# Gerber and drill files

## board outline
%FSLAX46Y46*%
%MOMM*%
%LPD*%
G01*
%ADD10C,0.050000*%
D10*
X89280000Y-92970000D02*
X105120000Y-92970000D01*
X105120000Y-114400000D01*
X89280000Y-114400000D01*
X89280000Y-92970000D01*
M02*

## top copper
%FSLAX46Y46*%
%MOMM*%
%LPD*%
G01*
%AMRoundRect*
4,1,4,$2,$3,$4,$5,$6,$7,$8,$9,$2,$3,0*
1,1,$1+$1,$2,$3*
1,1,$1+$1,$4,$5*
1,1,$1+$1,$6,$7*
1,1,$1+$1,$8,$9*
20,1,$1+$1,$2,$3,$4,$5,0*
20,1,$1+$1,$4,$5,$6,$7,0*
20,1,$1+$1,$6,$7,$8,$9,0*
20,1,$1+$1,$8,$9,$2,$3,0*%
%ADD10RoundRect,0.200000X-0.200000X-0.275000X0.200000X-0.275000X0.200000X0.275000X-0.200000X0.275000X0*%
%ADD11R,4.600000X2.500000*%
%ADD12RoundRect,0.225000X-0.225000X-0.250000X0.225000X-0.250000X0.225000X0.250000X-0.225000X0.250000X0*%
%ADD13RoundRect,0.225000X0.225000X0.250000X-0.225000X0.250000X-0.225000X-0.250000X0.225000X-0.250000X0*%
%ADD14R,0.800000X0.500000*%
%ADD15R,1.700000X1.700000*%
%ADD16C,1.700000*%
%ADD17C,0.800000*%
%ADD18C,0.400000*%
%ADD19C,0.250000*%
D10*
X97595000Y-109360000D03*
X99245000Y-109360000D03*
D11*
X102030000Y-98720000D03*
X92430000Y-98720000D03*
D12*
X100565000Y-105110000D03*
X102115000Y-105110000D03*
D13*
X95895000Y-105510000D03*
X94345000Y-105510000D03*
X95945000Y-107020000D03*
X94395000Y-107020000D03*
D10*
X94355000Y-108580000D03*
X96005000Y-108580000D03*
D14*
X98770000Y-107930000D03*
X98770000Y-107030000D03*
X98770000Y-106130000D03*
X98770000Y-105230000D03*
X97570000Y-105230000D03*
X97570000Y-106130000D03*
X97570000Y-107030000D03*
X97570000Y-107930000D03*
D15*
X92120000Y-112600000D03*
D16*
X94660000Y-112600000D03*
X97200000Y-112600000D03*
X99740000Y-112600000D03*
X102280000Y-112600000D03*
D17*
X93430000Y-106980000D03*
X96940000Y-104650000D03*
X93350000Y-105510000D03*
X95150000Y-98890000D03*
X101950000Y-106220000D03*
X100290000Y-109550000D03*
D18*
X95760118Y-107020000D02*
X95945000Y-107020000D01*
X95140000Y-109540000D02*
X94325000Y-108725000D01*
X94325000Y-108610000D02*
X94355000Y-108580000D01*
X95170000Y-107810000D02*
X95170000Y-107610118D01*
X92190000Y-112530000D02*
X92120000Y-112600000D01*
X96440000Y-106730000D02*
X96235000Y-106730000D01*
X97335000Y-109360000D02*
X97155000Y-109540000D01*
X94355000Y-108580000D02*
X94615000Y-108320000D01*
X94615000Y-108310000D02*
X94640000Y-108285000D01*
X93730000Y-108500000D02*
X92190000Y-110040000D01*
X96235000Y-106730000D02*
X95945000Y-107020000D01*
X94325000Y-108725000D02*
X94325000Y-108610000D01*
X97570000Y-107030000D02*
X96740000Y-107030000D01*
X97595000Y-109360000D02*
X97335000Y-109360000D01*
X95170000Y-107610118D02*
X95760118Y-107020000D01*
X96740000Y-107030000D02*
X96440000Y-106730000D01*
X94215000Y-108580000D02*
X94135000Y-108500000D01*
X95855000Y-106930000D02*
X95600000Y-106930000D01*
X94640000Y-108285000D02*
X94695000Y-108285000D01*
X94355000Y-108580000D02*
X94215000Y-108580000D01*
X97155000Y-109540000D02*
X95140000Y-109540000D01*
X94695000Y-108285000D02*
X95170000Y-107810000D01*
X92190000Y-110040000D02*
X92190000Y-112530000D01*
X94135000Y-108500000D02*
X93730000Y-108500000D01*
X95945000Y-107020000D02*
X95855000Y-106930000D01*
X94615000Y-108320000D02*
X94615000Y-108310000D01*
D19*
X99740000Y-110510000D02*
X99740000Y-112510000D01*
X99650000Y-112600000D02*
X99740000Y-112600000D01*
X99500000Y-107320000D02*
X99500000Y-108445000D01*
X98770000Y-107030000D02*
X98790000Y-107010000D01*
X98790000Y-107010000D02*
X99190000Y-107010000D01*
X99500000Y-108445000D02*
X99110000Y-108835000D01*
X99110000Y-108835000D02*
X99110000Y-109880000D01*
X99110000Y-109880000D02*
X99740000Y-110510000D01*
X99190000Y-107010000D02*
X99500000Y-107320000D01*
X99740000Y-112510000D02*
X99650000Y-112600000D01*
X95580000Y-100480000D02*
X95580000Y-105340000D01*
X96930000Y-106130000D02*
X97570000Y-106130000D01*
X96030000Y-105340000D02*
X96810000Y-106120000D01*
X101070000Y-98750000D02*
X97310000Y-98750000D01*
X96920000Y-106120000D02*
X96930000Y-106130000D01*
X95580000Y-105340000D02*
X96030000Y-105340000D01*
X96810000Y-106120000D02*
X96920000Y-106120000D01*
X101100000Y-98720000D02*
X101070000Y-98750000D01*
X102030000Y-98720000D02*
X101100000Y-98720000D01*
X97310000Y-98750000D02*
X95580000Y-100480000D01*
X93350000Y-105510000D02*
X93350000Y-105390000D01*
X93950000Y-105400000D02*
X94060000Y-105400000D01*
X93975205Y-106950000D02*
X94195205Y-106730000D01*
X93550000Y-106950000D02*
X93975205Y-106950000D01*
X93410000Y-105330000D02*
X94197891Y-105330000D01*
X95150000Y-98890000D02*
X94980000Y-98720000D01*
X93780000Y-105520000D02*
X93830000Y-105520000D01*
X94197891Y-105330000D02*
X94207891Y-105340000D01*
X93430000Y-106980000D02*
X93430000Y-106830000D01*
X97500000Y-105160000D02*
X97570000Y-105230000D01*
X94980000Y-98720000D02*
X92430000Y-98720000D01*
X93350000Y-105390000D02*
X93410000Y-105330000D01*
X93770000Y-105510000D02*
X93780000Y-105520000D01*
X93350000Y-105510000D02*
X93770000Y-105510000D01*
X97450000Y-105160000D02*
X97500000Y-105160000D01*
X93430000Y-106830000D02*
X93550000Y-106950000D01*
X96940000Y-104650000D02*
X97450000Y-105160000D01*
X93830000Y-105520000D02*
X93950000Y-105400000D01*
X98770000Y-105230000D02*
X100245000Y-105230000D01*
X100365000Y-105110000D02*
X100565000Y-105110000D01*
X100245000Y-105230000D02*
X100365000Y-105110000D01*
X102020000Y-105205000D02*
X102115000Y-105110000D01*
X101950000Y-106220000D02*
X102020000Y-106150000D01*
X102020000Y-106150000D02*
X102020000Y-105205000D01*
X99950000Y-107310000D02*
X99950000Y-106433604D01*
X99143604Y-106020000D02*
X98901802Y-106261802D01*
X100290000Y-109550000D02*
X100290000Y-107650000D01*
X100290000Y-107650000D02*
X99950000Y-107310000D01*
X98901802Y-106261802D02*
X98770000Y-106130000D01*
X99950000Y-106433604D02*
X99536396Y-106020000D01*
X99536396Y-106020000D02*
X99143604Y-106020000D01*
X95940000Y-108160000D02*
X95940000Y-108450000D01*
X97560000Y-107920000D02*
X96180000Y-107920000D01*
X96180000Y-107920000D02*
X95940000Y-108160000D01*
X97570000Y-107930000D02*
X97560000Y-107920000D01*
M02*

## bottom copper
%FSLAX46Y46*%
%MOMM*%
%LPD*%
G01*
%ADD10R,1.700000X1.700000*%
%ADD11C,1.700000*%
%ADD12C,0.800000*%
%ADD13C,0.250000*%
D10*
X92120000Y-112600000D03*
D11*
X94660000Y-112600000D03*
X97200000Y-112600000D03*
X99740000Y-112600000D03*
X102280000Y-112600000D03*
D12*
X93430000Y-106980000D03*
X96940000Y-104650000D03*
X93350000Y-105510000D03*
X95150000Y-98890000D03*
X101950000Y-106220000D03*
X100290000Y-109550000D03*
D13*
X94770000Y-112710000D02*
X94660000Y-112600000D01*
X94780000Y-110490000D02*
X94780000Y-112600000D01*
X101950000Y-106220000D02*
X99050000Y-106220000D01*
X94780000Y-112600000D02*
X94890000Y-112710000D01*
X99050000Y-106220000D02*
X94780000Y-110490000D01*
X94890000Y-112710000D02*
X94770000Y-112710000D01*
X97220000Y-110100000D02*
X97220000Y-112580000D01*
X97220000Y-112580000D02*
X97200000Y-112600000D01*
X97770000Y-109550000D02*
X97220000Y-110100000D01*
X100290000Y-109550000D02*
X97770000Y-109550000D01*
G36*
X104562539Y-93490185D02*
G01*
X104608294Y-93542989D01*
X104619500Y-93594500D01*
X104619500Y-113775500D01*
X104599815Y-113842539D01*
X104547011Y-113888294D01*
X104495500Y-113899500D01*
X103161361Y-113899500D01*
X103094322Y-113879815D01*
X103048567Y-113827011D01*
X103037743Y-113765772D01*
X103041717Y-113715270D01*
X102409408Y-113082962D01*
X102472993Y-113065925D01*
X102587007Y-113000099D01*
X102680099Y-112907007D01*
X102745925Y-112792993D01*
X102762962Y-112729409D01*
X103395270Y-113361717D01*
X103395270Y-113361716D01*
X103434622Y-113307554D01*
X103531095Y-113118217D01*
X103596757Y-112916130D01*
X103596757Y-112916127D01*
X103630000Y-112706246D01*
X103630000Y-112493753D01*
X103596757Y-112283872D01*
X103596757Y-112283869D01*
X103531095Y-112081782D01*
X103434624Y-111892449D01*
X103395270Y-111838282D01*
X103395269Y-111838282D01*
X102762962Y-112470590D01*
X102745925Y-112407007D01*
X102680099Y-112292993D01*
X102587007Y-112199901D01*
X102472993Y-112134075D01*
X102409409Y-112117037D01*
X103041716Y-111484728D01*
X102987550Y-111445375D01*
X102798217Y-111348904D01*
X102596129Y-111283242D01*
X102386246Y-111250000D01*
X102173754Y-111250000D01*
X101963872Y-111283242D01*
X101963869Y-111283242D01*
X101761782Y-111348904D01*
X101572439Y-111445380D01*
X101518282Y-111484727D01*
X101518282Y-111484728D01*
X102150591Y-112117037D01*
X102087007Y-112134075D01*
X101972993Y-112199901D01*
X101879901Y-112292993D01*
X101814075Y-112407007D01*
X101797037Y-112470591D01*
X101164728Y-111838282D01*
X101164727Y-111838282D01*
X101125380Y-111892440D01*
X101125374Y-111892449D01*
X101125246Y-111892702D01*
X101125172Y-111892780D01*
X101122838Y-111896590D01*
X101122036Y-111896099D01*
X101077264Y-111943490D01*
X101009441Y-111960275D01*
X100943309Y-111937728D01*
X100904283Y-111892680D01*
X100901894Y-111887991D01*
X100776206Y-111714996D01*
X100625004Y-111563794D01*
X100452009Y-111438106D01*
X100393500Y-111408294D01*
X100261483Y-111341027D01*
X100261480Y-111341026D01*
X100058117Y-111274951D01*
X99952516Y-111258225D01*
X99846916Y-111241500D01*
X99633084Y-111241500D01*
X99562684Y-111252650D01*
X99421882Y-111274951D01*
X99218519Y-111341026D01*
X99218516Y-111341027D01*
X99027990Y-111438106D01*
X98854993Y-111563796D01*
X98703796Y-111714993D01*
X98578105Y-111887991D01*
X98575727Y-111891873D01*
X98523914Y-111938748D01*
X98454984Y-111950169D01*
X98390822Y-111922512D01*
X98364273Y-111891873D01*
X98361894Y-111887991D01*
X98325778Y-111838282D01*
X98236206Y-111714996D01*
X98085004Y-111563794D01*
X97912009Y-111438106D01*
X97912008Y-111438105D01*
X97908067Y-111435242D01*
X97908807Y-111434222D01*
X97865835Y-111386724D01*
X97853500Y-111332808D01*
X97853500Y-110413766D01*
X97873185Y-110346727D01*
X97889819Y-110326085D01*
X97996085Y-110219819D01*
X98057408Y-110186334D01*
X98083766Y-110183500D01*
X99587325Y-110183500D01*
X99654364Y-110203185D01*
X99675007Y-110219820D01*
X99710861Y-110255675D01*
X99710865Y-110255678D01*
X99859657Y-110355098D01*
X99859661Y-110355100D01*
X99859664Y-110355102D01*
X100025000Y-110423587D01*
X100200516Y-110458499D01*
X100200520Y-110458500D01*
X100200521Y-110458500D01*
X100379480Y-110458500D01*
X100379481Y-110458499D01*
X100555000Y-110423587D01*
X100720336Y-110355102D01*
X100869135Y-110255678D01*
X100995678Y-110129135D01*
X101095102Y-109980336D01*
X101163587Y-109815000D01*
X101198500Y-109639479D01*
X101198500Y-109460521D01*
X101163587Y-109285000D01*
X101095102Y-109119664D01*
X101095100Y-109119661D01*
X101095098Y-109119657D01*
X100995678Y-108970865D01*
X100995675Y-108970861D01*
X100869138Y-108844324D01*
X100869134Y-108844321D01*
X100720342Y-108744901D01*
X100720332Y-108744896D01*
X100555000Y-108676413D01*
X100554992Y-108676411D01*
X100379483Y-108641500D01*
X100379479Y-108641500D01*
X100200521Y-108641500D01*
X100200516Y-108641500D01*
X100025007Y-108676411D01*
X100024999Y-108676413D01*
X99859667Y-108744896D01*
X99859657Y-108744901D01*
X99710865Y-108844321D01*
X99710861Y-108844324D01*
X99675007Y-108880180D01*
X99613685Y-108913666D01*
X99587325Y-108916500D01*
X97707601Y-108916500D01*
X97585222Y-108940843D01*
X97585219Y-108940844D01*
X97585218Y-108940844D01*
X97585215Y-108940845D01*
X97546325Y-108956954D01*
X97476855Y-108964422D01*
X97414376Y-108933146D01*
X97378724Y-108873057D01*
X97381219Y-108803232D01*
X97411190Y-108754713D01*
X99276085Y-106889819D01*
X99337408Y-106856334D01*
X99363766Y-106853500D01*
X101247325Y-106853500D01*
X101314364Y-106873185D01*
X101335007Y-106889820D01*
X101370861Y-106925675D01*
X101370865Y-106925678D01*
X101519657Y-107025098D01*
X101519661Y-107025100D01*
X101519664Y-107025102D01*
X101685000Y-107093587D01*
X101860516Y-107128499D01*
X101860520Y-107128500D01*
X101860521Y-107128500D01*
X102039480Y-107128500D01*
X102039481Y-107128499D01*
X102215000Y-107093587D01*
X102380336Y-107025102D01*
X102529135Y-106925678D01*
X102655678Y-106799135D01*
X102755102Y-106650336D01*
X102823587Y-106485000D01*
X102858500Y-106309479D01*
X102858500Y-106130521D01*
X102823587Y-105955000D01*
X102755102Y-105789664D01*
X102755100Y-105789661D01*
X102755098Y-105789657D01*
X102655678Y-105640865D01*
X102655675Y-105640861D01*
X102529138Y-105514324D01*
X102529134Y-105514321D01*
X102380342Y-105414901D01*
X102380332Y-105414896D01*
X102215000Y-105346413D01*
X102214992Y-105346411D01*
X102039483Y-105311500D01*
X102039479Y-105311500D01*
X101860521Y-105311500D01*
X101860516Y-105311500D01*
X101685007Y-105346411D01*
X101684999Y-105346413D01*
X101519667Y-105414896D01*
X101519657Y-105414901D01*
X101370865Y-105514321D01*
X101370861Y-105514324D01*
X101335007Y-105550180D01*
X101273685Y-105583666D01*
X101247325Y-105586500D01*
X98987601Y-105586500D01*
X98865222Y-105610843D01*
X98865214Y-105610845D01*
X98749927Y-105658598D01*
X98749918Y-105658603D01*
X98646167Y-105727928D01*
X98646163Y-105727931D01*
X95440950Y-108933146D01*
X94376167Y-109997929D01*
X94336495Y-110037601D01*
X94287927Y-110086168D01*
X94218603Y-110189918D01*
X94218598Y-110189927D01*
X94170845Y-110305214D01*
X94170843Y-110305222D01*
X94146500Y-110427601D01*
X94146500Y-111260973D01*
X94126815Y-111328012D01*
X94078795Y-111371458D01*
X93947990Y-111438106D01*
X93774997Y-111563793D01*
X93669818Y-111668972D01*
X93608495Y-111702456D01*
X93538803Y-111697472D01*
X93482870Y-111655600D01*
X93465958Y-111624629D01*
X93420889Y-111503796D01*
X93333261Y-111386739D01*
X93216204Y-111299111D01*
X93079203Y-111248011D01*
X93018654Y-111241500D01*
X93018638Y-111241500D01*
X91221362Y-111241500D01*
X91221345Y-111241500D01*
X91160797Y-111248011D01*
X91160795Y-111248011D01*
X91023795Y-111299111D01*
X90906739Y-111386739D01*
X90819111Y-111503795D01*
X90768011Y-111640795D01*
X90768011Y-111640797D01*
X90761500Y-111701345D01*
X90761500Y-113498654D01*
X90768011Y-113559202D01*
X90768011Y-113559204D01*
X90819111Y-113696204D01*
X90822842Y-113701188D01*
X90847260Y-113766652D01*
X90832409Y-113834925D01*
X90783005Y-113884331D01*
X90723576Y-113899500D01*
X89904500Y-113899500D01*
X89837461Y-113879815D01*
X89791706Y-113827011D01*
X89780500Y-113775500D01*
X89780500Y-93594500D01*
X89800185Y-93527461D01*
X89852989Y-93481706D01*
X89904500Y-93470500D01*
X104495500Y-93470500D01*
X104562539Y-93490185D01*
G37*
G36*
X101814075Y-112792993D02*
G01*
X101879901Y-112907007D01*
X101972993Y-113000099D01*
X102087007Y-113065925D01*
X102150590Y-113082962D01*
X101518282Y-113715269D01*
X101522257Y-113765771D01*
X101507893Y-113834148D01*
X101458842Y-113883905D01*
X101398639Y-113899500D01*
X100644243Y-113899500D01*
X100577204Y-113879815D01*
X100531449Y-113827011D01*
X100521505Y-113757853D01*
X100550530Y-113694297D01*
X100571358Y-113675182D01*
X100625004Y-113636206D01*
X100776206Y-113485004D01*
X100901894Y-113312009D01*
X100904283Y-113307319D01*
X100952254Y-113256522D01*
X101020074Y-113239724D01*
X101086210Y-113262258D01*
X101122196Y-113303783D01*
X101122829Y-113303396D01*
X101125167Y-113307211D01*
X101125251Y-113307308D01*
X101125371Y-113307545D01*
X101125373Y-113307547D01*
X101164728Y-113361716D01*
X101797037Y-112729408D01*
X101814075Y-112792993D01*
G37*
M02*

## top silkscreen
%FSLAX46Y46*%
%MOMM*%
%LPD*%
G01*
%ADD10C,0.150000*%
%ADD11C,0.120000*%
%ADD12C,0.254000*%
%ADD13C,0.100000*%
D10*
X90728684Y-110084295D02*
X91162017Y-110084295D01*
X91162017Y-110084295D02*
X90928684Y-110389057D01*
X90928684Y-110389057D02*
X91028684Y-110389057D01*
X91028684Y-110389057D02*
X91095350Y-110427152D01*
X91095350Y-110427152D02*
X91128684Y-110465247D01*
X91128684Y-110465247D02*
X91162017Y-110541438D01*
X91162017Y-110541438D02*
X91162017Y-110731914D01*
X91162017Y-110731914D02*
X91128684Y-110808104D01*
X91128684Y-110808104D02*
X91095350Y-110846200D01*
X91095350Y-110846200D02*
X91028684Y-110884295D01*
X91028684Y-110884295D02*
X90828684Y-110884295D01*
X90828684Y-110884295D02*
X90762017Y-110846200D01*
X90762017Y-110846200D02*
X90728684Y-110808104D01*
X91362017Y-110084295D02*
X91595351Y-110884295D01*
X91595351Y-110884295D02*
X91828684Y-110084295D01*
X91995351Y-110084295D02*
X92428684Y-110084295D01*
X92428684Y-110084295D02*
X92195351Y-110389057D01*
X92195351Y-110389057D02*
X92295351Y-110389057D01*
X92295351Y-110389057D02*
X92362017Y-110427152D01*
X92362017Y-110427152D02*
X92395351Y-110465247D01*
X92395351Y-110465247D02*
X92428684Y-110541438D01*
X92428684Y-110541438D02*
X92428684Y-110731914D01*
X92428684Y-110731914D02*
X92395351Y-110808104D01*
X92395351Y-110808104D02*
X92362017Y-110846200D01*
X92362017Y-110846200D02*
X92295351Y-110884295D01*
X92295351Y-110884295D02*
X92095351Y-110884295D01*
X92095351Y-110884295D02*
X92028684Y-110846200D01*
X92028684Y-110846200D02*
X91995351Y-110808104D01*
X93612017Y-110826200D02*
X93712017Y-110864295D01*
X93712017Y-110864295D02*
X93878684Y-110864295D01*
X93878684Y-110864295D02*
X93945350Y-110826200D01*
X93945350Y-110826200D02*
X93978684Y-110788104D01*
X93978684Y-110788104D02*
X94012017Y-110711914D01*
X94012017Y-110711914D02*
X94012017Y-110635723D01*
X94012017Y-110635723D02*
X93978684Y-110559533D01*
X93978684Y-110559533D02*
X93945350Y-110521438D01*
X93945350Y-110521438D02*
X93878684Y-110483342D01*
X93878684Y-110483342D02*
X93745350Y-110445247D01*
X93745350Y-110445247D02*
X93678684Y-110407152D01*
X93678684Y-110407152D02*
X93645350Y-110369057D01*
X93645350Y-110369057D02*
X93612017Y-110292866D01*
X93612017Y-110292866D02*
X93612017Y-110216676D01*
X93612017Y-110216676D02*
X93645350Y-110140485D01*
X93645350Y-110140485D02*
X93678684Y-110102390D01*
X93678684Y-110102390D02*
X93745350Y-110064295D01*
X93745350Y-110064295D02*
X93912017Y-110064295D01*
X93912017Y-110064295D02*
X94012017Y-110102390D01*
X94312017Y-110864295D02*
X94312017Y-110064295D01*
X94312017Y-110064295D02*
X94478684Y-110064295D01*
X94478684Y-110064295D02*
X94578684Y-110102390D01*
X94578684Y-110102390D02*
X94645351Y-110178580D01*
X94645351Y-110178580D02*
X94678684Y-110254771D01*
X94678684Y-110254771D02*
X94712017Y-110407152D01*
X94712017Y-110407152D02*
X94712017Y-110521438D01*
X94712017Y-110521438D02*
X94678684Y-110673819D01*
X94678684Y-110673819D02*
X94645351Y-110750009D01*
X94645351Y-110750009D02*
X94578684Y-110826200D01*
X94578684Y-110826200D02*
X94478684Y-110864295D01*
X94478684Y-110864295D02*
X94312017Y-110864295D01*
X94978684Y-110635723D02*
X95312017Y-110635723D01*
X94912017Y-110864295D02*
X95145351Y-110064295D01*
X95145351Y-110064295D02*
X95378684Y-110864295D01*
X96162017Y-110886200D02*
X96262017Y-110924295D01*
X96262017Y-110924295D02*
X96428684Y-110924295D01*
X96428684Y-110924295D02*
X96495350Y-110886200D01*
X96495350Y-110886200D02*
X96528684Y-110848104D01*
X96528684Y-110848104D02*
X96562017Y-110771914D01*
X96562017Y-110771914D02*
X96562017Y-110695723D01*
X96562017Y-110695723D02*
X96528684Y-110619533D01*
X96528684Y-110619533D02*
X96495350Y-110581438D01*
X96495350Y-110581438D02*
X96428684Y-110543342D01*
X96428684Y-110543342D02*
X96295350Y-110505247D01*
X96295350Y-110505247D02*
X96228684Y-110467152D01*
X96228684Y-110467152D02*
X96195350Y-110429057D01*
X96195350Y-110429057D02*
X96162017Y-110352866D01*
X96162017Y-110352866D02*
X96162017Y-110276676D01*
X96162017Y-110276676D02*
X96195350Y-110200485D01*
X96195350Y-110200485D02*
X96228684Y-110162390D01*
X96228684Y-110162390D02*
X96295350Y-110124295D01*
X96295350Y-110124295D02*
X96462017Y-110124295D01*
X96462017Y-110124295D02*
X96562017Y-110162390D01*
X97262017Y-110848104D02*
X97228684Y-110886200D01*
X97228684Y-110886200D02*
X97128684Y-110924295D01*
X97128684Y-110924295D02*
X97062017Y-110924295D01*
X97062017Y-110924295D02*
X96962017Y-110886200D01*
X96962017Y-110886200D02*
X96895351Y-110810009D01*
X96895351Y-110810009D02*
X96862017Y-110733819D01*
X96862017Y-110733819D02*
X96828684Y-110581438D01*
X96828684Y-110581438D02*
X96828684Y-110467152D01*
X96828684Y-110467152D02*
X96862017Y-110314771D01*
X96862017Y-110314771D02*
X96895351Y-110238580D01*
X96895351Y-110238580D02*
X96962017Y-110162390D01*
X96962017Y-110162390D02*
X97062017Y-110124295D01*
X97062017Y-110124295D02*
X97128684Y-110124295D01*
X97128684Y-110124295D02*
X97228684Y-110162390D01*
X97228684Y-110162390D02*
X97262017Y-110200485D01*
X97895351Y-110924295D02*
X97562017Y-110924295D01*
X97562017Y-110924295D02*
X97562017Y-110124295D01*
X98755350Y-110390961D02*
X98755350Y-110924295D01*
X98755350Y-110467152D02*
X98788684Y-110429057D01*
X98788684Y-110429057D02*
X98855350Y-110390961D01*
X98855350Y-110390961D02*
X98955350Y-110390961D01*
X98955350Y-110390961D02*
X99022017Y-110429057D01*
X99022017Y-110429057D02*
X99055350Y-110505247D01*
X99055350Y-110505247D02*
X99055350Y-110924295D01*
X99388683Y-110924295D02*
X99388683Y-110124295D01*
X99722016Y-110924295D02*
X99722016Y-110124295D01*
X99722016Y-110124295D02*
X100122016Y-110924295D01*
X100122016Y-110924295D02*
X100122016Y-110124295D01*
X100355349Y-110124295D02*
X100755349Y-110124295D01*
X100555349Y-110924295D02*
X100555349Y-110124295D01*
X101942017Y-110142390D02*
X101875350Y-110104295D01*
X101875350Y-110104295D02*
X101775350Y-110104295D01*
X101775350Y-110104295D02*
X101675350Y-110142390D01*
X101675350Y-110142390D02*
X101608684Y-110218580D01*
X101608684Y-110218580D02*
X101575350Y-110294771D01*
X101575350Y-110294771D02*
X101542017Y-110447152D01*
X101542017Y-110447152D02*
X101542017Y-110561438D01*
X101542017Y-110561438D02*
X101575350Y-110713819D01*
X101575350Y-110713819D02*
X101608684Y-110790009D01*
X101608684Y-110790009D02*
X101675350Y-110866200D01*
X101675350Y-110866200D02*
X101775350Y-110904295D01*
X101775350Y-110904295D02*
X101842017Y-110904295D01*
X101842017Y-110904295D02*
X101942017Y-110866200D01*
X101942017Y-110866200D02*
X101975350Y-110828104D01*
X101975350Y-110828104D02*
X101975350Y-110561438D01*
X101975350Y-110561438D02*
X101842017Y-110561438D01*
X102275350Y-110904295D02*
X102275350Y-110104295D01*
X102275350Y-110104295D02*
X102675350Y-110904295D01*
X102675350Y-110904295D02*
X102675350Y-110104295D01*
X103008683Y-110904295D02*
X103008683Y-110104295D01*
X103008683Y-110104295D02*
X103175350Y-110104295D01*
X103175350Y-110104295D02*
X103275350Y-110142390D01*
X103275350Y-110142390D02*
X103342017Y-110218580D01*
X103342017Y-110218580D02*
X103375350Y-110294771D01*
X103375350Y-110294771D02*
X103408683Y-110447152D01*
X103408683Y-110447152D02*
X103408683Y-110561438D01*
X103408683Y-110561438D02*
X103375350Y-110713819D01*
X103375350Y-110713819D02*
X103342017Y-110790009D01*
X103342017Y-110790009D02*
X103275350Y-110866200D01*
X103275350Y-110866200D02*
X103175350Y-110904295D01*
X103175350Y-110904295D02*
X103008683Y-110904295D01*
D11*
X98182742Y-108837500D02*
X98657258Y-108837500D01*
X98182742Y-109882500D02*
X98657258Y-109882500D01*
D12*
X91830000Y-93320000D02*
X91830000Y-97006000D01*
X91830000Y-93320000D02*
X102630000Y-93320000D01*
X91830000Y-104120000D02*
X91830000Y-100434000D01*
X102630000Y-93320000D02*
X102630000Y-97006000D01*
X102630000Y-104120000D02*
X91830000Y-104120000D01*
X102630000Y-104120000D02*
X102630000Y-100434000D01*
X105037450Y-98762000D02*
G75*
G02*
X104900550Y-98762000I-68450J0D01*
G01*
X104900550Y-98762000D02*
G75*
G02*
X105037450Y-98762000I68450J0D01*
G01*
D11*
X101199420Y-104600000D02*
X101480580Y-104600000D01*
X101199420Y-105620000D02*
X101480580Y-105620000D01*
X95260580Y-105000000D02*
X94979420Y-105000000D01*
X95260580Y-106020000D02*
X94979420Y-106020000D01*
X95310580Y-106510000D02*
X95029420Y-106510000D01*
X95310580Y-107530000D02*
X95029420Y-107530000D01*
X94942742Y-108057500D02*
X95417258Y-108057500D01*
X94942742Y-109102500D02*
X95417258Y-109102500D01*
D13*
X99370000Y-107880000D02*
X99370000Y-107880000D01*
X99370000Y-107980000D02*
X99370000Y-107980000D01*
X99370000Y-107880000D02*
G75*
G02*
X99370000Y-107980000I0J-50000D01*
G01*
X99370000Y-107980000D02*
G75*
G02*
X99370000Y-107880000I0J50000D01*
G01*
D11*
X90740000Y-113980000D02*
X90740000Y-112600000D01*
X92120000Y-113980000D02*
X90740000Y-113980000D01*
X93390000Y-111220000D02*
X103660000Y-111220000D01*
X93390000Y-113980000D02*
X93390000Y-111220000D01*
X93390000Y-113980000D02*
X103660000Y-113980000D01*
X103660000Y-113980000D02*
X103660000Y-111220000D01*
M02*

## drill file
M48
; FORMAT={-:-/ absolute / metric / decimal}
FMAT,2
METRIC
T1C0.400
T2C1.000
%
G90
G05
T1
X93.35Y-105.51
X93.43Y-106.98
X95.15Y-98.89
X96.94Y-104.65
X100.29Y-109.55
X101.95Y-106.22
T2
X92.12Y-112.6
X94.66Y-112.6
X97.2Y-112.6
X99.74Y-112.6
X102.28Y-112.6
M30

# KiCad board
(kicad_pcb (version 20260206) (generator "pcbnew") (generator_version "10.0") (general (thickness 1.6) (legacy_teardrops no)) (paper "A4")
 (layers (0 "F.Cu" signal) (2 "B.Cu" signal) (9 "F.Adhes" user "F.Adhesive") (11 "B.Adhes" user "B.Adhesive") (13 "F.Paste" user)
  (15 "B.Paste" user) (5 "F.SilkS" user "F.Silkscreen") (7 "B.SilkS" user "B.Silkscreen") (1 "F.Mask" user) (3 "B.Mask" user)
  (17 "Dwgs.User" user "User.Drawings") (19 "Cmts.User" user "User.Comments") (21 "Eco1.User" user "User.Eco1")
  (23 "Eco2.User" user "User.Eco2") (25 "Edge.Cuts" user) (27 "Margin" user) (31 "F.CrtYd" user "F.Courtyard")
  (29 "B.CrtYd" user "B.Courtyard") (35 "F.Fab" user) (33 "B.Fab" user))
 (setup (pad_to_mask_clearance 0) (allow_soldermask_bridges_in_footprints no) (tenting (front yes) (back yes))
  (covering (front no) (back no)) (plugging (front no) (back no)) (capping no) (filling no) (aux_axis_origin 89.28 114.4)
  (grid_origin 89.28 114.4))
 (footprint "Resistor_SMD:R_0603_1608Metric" (layer "F.Cu") (at 98.42 109.36)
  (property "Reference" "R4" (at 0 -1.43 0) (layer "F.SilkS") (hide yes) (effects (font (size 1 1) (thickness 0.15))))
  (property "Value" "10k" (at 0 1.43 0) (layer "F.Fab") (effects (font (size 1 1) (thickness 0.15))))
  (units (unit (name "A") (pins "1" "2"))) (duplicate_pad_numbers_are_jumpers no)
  (fp_line (start -0.237258 -0.5225) (end 0.237258 -0.5225) (stroke (width 0.12) (type solid)) (layer "F.SilkS"))
  (fp_line (start -0.237258 0.5225) (end 0.237258 0.5225) (stroke (width 0.12) (type solid)) (layer "F.SilkS"))
  (pad "1" smd roundrect (at -0.825 0) (size 0.8 0.95) (layers "F.Cu" "F.Mask" "F.Paste") (roundrect_rratio 0.25) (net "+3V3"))
  (pad "2" smd roundrect (at 0.825 0) (size 0.8 0.95) (layers "F.Cu" "F.Mask" "F.Paste") (roundrect_rratio 0.25) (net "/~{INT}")))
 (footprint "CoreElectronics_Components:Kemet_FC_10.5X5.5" (layer "F.Cu") (at 97.23 98.72 180)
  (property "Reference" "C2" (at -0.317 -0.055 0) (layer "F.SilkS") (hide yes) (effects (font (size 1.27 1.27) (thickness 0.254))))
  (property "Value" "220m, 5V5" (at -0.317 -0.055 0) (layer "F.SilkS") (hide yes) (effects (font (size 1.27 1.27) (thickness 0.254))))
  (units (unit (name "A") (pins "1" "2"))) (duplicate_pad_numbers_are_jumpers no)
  (fp_line (start 5.4 5.4) (end 5.4 1.714) (stroke (width 0.254) (type solid)) (layer "F.SilkS"))
  (fp_line (start 5.4 5.4) (end -5.4 5.4) (stroke (width 0.254) (type solid)) (layer "F.SilkS"))
  (fp_line (start 5.4 -5.4) (end 5.4 -1.714) (stroke (width 0.254) (type solid)) (layer "F.SilkS"))
  (fp_line (start -5.4 5.4) (end -5.4 1.714) (stroke (width 0.254) (type solid)) (layer "F.SilkS"))
  (fp_line (start -5.4 -5.4) (end 5.4 -5.4) (stroke (width 0.254) (type solid)) (layer "F.SilkS"))
  (fp_line (start -5.4 -5.4) (end -5.4 -1.714) (stroke (width 0.254) (type solid)) (layer "F.SilkS"))
  (fp_circle (center -7.739 -0.042) (end -7.739 0.02645) (stroke (width 0.254) (type solid)) (fill no) (layer "F.SilkS"))
  (pad "1" smd rect (at -4.8 0 270) (size 2.5 4.6) (layers "F.Cu" "F.Mask" "F.Paste") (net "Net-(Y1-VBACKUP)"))
  (pad "2" smd rect (at 4.8 0 270) (size 2.5 4.6) (layers "F.Cu" "F.Mask" "F.Paste") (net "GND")))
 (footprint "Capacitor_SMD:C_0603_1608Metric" (layer "F.Cu") (at 101.34 105.11)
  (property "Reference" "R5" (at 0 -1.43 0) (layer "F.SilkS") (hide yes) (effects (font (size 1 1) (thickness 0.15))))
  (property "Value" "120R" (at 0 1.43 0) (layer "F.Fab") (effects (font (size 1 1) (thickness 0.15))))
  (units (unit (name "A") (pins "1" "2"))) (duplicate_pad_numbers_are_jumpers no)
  (fp_line (start -0.14058 -0.51) (end 0.14058 -0.51) (stroke (width 0.12) (type solid)) (layer "F.SilkS"))
  (fp_line (start -0.14058 0.51) (end 0.14058 0.51) (stroke (width 0.12) (type solid)) (layer "F.SilkS"))
  (pad "1" smd roundrect (at -0.775 0) (size 0.9 0.95) (layers "F.Cu" "F.Mask" "F.Paste") (roundrect_rratio 0.25) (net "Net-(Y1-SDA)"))
  (pad "2" smd roundrect (at 0.775 0) (size 0.9 0.95) (layers "F.Cu" "F.Mask" "F.Paste") (roundrect_rratio 0.25) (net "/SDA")))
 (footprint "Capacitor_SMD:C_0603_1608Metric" (layer "F.Cu") (at 95.12 105.51 180)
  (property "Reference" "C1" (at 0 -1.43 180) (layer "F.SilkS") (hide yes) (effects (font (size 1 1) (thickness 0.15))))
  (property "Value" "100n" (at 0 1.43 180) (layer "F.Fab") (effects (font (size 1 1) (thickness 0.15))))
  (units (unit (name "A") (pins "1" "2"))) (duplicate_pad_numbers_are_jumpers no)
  (fp_line (start -0.14058 0.51) (end 0.14058 0.51) (stroke (width 0.12) (type solid)) (layer "F.SilkS"))
  (fp_line (start -0.14058 -0.51) (end 0.14058 -0.51) (stroke (width 0.12) (type solid)) (layer "F.SilkS"))
  (pad "1" smd roundrect (at -0.775 0 180) (size 0.9 0.95) (layers "F.Cu" "F.Mask" "F.Paste") (roundrect_rratio 0.25)
   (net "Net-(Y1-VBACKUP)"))
  (pad "2" smd roundrect (at 0.775 0 180) (size 0.9 0.95) (layers "F.Cu" "F.Mask" "F.Paste") (roundrect_rratio 0.25) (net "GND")))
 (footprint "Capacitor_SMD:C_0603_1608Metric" (layer "F.Cu") (at 95.17 107.02 180)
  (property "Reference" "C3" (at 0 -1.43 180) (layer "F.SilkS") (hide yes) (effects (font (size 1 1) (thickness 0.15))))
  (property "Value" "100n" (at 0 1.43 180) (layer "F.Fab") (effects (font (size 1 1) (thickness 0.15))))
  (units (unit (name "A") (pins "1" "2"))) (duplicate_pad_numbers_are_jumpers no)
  (fp_line (start -0.14058 0.51) (end 0.14058 0.51) (stroke (width 0.12) (type solid)) (layer "F.SilkS"))
  (fp_line (start -0.14058 -0.51) (end 0.14058 -0.51) (stroke (width 0.12) (type solid)) (layer "F.SilkS"))
  (pad "1" smd roundrect (at -0.775 0 180) (size 0.9 0.95) (layers "F.Cu" "F.Mask" "F.Paste") (roundrect_rratio 0.25) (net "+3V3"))
  (pad "2" smd roundrect (at 0.775 0 180) (size 0.9 0.95) (layers "F.Cu" "F.Mask" "F.Paste") (roundrect_rratio 0.25) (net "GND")))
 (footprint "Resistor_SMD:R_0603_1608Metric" (layer "F.Cu") (at 95.18 108.58)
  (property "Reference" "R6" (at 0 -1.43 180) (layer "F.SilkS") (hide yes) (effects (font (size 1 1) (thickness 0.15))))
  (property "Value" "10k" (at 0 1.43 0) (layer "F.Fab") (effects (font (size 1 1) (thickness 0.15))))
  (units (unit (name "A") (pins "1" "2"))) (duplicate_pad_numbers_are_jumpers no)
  (fp_line (start -0.237258 -0.5225) (end 0.237258 -0.5225) (stroke (width 0.12) (type solid)) (layer "F.SilkS"))
  (fp_line (start -0.237258 0.5225) (end 0.237258 0.5225) (stroke (width 0.12) (type solid)) (layer "F.SilkS"))
  (pad "1" smd roundrect (at -0.825 0) (size 0.8 0.95) (layers "F.Cu" "F.Mask" "F.Paste") (roundrect_rratio 0.25) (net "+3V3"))
  (pad "2" smd roundrect (at 0.825 0) (size 0.8 0.95) (layers "F.Cu" "F.Mask" "F.Paste") (roundrect_rratio 0.25) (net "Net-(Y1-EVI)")))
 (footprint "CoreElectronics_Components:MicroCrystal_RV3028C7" (layer "F.Cu") (at 98.17 106.58 90)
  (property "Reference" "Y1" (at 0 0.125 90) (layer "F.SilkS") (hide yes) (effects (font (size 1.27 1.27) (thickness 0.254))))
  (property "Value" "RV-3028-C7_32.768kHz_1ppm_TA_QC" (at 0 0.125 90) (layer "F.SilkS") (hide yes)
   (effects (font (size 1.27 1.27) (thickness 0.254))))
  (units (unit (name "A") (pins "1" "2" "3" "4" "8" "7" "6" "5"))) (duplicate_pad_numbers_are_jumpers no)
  (fp_line (start -1.3 1.2) (end -1.3 1.2) (stroke (width 0.1) (type solid)) (layer "F.SilkS"))
  (fp_line (start -1.4 1.2) (end -1.4 1.2) (stroke (width 0.1) (type solid)) (layer "F.SilkS"))
  (fp_arc (start -1.3 1.2) (mid -1.35 1.25) (end -1.4 1.2) (stroke (width 0.1) (type solid)) (layer "F.SilkS"))
  (fp_arc (start -1.4 1.2) (mid -1.35 1.15) (end -1.3 1.2) (stroke (width 0.1) (type solid)) (layer "F.SilkS"))
  (pad "1" smd rect (at -1.35 0.6 90) (size 0.5 0.8) (layers "F.Cu" "F.Mask" "F.Paste") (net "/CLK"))
  (pad "2" smd rect (at -0.45 0.6 90) (size 0.5 0.8) (layers "F.Cu" "F.Mask" "F.Paste") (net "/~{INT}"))
  (pad "3" smd rect (at 0.45 0.6 90) (size 0.5 0.8) (layers "F.Cu" "F.Mask" "F.Paste") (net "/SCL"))
  (pad "4" smd rect (at 1.35 0.6 90) (size 0.5 0.8) (layers "F.Cu" "F.Mask" "F.Paste") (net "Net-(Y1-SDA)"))
  (pad "5" smd rect (at 1.35 -0.6 90) (size 0.5 0.8) (layers "F.Cu" "F.Mask" "F.Paste") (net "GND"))
  (pad "6" smd rect (at 0.45 -0.6 90) (size 0.5 0.8) (layers "F.Cu" "F.Mask" "F.Paste") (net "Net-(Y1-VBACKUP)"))
  (pad "7" smd rect (at -0.45 -0.6 90) (size 0.5 0.8) (layers "F.Cu" "F.Mask" "F.Paste") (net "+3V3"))
  (pad "8" smd rect (at -1.35 -0.6 90) (size 0.5 0.8) (layers "F.Cu" "F.Mask" "F.Paste") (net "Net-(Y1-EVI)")))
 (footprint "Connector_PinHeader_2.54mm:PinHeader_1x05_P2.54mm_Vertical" (layer "F.Cu") (at 92.12 112.6 90)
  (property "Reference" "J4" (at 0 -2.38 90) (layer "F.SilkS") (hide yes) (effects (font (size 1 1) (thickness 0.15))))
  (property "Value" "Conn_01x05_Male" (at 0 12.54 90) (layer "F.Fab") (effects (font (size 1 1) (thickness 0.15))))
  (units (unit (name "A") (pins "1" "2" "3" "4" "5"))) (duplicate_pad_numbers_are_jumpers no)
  (fp_line (start -1.38 -1.38) (end 0 -1.38) (stroke (width 0.12) (type solid)) (layer "F.SilkS"))
  (fp_line (start -1.38 0) (end -1.38 -1.38) (stroke (width 0.12) (type solid)) (layer "F.SilkS"))
  (fp_line (start 1.38 1.27) (end 1.38 11.54) (stroke (width 0.12) (type solid)) (layer "F.SilkS"))
  (fp_line (start -1.38 1.27) (end 1.38 1.27) (stroke (width 0.12) (type solid)) (layer "F.SilkS"))
  (fp_line (start -1.38 1.27) (end -1.38 11.54) (stroke (width 0.12) (type solid)) (layer "F.SilkS"))
  (fp_line (start -1.38 11.54) (end 1.38 11.54) (stroke (width 0.12) (type solid)) (layer "F.SilkS"))
  (pad "1" thru_hole rect (at 0 0 90) (size 1.7 1.7) (drill 1) (layers "*.Cu" "*.Mask") (remove_unused_layers no) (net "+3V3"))
  (pad "2" thru_hole circle (at 0 2.54 90) (size 1.7 1.7) (drill 1) (layers "*.Cu" "*.Mask") (remove_unused_layers no) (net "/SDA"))
  (pad "3" thru_hole circle (at 0 5.08 90) (size 1.7 1.7) (drill 1) (layers "*.Cu" "*.Mask") (remove_unused_layers no) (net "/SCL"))
  (pad "4" thru_hole circle (at 0 7.62 90) (size 1.7 1.7) (drill 1) (layers "*.Cu" "*.Mask") (remove_unused_layers no) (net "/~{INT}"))
  (pad "5" thru_hole circle (at 0 10.16 90) (size 1.7 1.7) (drill 1) (layers "*.Cu" "*.Mask") (remove_unused_layers no) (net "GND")))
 (gr_rect (start 89.28 92.97) (end 105.12 114.4) (stroke (width 0.05) (type default)) (fill no) (layer "Edge.Cuts"))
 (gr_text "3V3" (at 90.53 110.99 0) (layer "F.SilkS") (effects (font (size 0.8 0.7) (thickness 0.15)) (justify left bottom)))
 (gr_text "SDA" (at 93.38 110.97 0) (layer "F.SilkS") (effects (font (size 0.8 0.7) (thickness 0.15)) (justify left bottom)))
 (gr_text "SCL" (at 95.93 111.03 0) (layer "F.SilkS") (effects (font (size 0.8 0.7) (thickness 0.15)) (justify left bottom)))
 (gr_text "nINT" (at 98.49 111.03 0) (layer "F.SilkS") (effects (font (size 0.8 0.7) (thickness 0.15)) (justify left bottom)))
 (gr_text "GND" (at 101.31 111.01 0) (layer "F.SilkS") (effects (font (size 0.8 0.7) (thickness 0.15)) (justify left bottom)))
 (segment (start 95.760118 107.02) (end 95.945 107.02) (width 0.4) (layer "F.Cu") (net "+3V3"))
 (segment (start 95.14 109.54) (end 94.325 108.725) (width 0.4) (layer "F.Cu") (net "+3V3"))
 (segment (start 94.325 108.61) (end 94.355 108.58) (width 0.4) (layer "F.Cu") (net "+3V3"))
 (segment (start 95.17 107.81) (end 95.17 107.610118) (width 0.4) (layer "F.Cu") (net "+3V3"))
 (segment (start 92.19 112.53) (end 92.12 112.6) (width 0.4) (layer "F.Cu") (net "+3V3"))
 (segment (start 96.44 106.73) (end 96.235 106.73) (width 0.4) (layer "F.Cu") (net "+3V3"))
 (segment (start 97.335 109.36) (end 97.155 109.54) (width 0.4) (layer "F.Cu") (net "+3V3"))
 (segment (start 94.355 108.58) (end 94.615 108.32) (width 0.4) (layer "F.Cu") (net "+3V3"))
 (segment (start 94.615 108.31) (end 94.64 108.285) (width 0.4) (layer "F.Cu") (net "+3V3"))
 (segment (start 93.73 108.5) (end 92.19 110.04) (width 0.4) (layer "F.Cu") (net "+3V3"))
 (segment (start 96.235 106.73) (end 95.945 107.02) (width 0.4) (layer "F.Cu") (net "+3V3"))
 (segment (start 94.325 108.725) (end 94.325 108.61) (width 0.4) (layer "F.Cu") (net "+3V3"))
 (segment (start 97.57 107.03) (end 96.74 107.03) (width 0.4) (layer "F.Cu") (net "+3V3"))
 (segment (start 97.595 109.36) (end 97.335 109.36) (width 0.4) (layer "F.Cu") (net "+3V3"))
 (segment (start 95.17 107.610118) (end 95.760118 107.02) (width 0.4) (layer "F.Cu") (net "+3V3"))
 (segment (start 96.74 107.03) (end 96.44 106.73) (width 0.4) (layer "F.Cu") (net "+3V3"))
 (segment (start 94.215 108.58) (end 94.135 108.5) (width 0.4) (layer "F.Cu") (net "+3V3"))
 (segment (start 95.855 106.93) (end 95.6 106.93) (width 0.4) (layer "F.Cu") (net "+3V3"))
 (segment (start 94.64 108.285) (end 94.695 108.285) (width 0.4) (layer "F.Cu") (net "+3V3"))
 (segment (start 94.355 108.58) (end 94.215 108.58) (width 0.4) (layer "F.Cu") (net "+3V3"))
 (segment (start 97.155 109.54) (end 95.14 109.54) (width 0.4) (layer "F.Cu") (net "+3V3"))
 (segment (start 94.695 108.285) (end 95.17 107.81) (width 0.4) (layer "F.Cu") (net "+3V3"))
 (segment (start 92.19 110.04) (end 92.19 112.53) (width 0.4) (layer "F.Cu") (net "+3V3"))
 (segment (start 94.135 108.5) (end 93.73 108.5) (width 0.4) (layer "F.Cu") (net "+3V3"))
 (segment (start 95.945 107.02) (end 95.855 106.93) (width 0.4) (layer "F.Cu") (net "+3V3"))
 (segment (start 94.615 108.32) (end 94.615 108.31) (width 0.4) (layer "F.Cu") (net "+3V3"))
 (segment (start 99.74 110.51) (end 99.74 112.51) (width 0.25) (layer "F.Cu") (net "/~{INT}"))
 (segment (start 99.65 112.6) (end 99.74 112.6) (width 0.25) (layer "F.Cu") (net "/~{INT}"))
 (segment (start 99.5 107.32) (end 99.5 108.445) (width 0.25) (layer "F.Cu") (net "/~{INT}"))
 (segment (start 98.77 107.03) (end 98.79 107.01) (width 0.25) (layer "F.Cu") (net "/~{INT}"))
 (segment (start 98.79 107.01) (end 99.19 107.01) (width 0.25) (layer "F.Cu") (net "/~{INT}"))
 (segment (start 99.5 108.445) (end 99.11 108.835) (width 0.25) (layer "F.Cu") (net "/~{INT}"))
 (segment (start 99.11 108.835) (end 99.11 109.88) (width 0.25) (layer "F.Cu") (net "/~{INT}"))
 (segment (start 99.11 109.88) (end 99.74 110.51) (width 0.25) (layer "F.Cu") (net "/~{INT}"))
 (segment (start 99.19 107.01) (end 99.5 107.32) (width 0.25) (layer "F.Cu") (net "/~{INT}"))
 (segment (start 99.74 112.51) (end 99.65 112.6) (width 0.25) (layer "F.Cu") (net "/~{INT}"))
 (segment (start 95.58 100.48) (end 95.58 105.34) (width 0.25) (layer "F.Cu") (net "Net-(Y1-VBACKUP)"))
 (segment (start 96.93 106.13) (end 97.57 106.13) (width 0.25) (layer "F.Cu") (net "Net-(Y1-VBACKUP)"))
 (segment (start 96.03 105.34) (end 96.81 106.12) (width 0.25) (layer "F.Cu") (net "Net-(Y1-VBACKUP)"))
 (segment (start 101.07 98.75) (end 97.31 98.75) (width 0.25) (layer "F.Cu") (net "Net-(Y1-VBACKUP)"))
 (segment (start 96.92 106.12) (end 96.93 106.13) (width 0.25) (layer "F.Cu") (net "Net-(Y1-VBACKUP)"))
 (segment (start 95.58 105.34) (end 96.03 105.34) (width 0.25) (layer "F.Cu") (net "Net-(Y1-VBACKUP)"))
 (segment (start 96.81 106.12) (end 96.92 106.12) (width 0.25) (layer "F.Cu") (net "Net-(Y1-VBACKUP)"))
 (segment (start 101.1 98.72) (end 101.07 98.75) (width 0.25) (layer "F.Cu") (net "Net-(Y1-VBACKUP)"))
 (segment (start 102.03 98.72) (end 101.1 98.72) (width 0.25) (layer "F.Cu") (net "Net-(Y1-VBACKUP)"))
 (segment (start 97.31 98.75) (end 95.58 100.48) (width 0.25) (layer "F.Cu") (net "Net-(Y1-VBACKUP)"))
 (segment (start 93.35 105.51) (end 93.35 105.39) (width 0.25) (layer "F.Cu") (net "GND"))
 (segment (start 93.95 105.4) (end 94.06 105.4) (width 0.25) (layer "F.Cu") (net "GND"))
 (segment (start 93.975205 106.95) (end 94.195205 106.73) (width 0.25) (layer "F.Cu") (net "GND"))
 (segment (start 93.55 106.95) (end 93.975205 106.95) (width 0.25) (layer "F.Cu") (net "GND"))
 (segment (start 93.41 105.33) (end 94.197891 105.33) (width 0.25) (layer "F.Cu") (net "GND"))
 (segment (start 95.15 98.89) (end 94.98 98.72) (width 0.25) (layer "F.Cu") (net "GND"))
 (segment (start 93.78 105.52) (end 93.83 105.52) (width 0.25) (layer "F.Cu") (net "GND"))
 (segment (start 94.197891 105.33) (end 94.207891 105.34) (width 0.25) (layer "F.Cu") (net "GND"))
 (segment (start 93.43 106.98) (end 93.43 106.83) (width 0.25) (layer "F.Cu") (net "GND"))
 (segment (start 97.5 105.16) (end 97.57 105.23) (width 0.25) (layer "F.Cu") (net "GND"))
 (segment (start 94.98 98.72) (end 92.43 98.72) (width 0.25) (layer "F.Cu") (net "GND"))
 (segment (start 93.35 105.39) (end 93.41 105.33) (width 0.25) (layer "F.Cu") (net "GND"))
 (segment (start 93.77 105.51) (end 93.78 105.52) (width 0.25) (layer "F.Cu") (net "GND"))
 (segment (start 93.35 105.51) (end 93.77 105.51) (width 0.25) (layer "F.Cu") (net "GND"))
 (segment (start 97.45 105.16) (end 97.5 105.16) (width 0.25) (layer "F.Cu") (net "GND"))
 (segment (start 93.43 106.83) (end 93.55 106.95) (width 0.25) (layer "F.Cu") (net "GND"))
 (segment (start 96.94 104.65) (end 97.45 105.16) (width 0.25) (layer "F.Cu") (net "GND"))
 (segment (start 93.83 105.52) (end 93.95 105.4) (width 0.25) (layer "F.Cu") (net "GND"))
 (via (at 93.43 106.98) (size 0.8) (drill 0.4) (layers "F.Cu" "B.Cu") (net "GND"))
 (via (at 96.94 104.65) (size 0.8) (drill 0.4) (layers "F.Cu" "B.Cu") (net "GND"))
 (via (at 93.35 105.51) (size 0.8) (drill 0.4) (layers "F.Cu" "B.Cu") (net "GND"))
 (via (at 95.15 98.89) (size 0.8) (drill 0.4) (layers "F.Cu" "B.Cu") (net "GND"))
 (segment (start 98.77 105.23) (end 100.245 105.23) (width 0.25) (layer "F.Cu") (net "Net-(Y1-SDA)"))
 (segment (start 100.365 105.11) (end 100.565 105.11) (width 0.25) (layer "F.Cu") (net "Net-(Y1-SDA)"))
 (segment (start 100.245 105.23) (end 100.365 105.11) (width 0.25) (layer "F.Cu") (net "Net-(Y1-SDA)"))
 (segment (start 102.02 105.205) (end 102.115 105.11) (width 0.25) (layer "F.Cu") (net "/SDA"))
 (segment (start 101.95 106.22) (end 102.02 106.15) (width 0.25) (layer "F.Cu") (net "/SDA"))
 (segment (start 102.02 106.15) (end 102.02 105.205) (width 0.25) (layer "F.Cu") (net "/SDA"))
 (via (at 101.95 106.22) (size 0.8) (drill 0.4) (layers "F.Cu" "B.Cu") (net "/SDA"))
 (segment (start 94.77 112.71) (end 94.66 112.6) (width 0.25) (layer "B.Cu") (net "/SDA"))
 (segment (start 94.78 110.49) (end 94.78 112.6) (width 0.25) (layer "B.Cu") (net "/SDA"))
 (segment (start 101.95 106.22) (end 99.05 106.22) (width 0.25) (layer "B.Cu") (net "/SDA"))
 (segment (start 94.78 112.6) (end 94.89 112.71) (width 0.25) (layer "B.Cu") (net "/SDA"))
 (segment (start 99.05 106.22) (end 94.78 110.49) (width 0.25) (layer "B.Cu") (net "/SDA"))
 (segment (start 94.89 112.71) (end 94.77 112.71) (width 0.25) (layer "B.Cu") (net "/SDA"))
 (segment (start 99.95 107.31) (end 99.95 106.433604) (width 0.25) (layer "F.Cu") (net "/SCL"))
 (segment (start 99.143604 106.02) (end 98.901802 106.261802) (width 0.25) (layer "F.Cu") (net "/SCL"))
 (segment (start 100.29 109.55) (end 100.29 107.65) (width 0.25) (layer "F.Cu") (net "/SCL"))
 (segment (start 100.29 107.65) (end 99.95 107.31) (width 0.25) (layer "F.Cu") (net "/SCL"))
 (segment (start 98.901802 106.261802) (end 98.77 106.13) (width 0.25) (layer "F.Cu") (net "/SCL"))
 (segment (start 99.95 106.433604) (end 99.536396 106.02) (width 0.25) (layer "F.Cu") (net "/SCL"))
 (segment (start 99.536396 106.02) (end 99.143604 106.02) (width 0.25) (layer "F.Cu") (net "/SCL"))
 (via (at 100.29 109.55) (size 0.8) (drill 0.4) (layers "F.Cu" "B.Cu") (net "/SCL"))
 (segment (start 97.22 110.1) (end 97.22 112.58) (width 0.25) (layer "B.Cu") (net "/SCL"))
 (segment (start 97.22 112.58) (end 97.2 112.6) (width 0.25) (layer "B.Cu") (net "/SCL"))
 (segment (start 97.77 109.55) (end 97.22 110.1) (width 0.25) (layer "B.Cu") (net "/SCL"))
 (segment (start 100.29 109.55) (end 97.77 109.55) (width 0.25) (layer "B.Cu") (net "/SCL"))
 (segment (start 95.94 108.16) (end 95.94 108.45) (width 0.25) (layer "F.Cu") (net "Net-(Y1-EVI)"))
 (segment (start 97.56 107.92) (end 96.18 107.92) (width 0.25) (layer "F.Cu") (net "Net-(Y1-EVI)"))
 (segment (start 96.18 107.92) (end 95.94 108.16) (width 0.25) (layer "F.Cu") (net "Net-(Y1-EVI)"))
 (segment (start 97.57 107.93) (end 97.56 107.92) (width 0.25) (layer "F.Cu") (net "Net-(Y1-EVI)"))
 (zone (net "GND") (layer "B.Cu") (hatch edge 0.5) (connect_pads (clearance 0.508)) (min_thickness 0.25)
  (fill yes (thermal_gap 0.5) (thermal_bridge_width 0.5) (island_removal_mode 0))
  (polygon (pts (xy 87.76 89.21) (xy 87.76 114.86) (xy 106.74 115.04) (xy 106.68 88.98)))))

